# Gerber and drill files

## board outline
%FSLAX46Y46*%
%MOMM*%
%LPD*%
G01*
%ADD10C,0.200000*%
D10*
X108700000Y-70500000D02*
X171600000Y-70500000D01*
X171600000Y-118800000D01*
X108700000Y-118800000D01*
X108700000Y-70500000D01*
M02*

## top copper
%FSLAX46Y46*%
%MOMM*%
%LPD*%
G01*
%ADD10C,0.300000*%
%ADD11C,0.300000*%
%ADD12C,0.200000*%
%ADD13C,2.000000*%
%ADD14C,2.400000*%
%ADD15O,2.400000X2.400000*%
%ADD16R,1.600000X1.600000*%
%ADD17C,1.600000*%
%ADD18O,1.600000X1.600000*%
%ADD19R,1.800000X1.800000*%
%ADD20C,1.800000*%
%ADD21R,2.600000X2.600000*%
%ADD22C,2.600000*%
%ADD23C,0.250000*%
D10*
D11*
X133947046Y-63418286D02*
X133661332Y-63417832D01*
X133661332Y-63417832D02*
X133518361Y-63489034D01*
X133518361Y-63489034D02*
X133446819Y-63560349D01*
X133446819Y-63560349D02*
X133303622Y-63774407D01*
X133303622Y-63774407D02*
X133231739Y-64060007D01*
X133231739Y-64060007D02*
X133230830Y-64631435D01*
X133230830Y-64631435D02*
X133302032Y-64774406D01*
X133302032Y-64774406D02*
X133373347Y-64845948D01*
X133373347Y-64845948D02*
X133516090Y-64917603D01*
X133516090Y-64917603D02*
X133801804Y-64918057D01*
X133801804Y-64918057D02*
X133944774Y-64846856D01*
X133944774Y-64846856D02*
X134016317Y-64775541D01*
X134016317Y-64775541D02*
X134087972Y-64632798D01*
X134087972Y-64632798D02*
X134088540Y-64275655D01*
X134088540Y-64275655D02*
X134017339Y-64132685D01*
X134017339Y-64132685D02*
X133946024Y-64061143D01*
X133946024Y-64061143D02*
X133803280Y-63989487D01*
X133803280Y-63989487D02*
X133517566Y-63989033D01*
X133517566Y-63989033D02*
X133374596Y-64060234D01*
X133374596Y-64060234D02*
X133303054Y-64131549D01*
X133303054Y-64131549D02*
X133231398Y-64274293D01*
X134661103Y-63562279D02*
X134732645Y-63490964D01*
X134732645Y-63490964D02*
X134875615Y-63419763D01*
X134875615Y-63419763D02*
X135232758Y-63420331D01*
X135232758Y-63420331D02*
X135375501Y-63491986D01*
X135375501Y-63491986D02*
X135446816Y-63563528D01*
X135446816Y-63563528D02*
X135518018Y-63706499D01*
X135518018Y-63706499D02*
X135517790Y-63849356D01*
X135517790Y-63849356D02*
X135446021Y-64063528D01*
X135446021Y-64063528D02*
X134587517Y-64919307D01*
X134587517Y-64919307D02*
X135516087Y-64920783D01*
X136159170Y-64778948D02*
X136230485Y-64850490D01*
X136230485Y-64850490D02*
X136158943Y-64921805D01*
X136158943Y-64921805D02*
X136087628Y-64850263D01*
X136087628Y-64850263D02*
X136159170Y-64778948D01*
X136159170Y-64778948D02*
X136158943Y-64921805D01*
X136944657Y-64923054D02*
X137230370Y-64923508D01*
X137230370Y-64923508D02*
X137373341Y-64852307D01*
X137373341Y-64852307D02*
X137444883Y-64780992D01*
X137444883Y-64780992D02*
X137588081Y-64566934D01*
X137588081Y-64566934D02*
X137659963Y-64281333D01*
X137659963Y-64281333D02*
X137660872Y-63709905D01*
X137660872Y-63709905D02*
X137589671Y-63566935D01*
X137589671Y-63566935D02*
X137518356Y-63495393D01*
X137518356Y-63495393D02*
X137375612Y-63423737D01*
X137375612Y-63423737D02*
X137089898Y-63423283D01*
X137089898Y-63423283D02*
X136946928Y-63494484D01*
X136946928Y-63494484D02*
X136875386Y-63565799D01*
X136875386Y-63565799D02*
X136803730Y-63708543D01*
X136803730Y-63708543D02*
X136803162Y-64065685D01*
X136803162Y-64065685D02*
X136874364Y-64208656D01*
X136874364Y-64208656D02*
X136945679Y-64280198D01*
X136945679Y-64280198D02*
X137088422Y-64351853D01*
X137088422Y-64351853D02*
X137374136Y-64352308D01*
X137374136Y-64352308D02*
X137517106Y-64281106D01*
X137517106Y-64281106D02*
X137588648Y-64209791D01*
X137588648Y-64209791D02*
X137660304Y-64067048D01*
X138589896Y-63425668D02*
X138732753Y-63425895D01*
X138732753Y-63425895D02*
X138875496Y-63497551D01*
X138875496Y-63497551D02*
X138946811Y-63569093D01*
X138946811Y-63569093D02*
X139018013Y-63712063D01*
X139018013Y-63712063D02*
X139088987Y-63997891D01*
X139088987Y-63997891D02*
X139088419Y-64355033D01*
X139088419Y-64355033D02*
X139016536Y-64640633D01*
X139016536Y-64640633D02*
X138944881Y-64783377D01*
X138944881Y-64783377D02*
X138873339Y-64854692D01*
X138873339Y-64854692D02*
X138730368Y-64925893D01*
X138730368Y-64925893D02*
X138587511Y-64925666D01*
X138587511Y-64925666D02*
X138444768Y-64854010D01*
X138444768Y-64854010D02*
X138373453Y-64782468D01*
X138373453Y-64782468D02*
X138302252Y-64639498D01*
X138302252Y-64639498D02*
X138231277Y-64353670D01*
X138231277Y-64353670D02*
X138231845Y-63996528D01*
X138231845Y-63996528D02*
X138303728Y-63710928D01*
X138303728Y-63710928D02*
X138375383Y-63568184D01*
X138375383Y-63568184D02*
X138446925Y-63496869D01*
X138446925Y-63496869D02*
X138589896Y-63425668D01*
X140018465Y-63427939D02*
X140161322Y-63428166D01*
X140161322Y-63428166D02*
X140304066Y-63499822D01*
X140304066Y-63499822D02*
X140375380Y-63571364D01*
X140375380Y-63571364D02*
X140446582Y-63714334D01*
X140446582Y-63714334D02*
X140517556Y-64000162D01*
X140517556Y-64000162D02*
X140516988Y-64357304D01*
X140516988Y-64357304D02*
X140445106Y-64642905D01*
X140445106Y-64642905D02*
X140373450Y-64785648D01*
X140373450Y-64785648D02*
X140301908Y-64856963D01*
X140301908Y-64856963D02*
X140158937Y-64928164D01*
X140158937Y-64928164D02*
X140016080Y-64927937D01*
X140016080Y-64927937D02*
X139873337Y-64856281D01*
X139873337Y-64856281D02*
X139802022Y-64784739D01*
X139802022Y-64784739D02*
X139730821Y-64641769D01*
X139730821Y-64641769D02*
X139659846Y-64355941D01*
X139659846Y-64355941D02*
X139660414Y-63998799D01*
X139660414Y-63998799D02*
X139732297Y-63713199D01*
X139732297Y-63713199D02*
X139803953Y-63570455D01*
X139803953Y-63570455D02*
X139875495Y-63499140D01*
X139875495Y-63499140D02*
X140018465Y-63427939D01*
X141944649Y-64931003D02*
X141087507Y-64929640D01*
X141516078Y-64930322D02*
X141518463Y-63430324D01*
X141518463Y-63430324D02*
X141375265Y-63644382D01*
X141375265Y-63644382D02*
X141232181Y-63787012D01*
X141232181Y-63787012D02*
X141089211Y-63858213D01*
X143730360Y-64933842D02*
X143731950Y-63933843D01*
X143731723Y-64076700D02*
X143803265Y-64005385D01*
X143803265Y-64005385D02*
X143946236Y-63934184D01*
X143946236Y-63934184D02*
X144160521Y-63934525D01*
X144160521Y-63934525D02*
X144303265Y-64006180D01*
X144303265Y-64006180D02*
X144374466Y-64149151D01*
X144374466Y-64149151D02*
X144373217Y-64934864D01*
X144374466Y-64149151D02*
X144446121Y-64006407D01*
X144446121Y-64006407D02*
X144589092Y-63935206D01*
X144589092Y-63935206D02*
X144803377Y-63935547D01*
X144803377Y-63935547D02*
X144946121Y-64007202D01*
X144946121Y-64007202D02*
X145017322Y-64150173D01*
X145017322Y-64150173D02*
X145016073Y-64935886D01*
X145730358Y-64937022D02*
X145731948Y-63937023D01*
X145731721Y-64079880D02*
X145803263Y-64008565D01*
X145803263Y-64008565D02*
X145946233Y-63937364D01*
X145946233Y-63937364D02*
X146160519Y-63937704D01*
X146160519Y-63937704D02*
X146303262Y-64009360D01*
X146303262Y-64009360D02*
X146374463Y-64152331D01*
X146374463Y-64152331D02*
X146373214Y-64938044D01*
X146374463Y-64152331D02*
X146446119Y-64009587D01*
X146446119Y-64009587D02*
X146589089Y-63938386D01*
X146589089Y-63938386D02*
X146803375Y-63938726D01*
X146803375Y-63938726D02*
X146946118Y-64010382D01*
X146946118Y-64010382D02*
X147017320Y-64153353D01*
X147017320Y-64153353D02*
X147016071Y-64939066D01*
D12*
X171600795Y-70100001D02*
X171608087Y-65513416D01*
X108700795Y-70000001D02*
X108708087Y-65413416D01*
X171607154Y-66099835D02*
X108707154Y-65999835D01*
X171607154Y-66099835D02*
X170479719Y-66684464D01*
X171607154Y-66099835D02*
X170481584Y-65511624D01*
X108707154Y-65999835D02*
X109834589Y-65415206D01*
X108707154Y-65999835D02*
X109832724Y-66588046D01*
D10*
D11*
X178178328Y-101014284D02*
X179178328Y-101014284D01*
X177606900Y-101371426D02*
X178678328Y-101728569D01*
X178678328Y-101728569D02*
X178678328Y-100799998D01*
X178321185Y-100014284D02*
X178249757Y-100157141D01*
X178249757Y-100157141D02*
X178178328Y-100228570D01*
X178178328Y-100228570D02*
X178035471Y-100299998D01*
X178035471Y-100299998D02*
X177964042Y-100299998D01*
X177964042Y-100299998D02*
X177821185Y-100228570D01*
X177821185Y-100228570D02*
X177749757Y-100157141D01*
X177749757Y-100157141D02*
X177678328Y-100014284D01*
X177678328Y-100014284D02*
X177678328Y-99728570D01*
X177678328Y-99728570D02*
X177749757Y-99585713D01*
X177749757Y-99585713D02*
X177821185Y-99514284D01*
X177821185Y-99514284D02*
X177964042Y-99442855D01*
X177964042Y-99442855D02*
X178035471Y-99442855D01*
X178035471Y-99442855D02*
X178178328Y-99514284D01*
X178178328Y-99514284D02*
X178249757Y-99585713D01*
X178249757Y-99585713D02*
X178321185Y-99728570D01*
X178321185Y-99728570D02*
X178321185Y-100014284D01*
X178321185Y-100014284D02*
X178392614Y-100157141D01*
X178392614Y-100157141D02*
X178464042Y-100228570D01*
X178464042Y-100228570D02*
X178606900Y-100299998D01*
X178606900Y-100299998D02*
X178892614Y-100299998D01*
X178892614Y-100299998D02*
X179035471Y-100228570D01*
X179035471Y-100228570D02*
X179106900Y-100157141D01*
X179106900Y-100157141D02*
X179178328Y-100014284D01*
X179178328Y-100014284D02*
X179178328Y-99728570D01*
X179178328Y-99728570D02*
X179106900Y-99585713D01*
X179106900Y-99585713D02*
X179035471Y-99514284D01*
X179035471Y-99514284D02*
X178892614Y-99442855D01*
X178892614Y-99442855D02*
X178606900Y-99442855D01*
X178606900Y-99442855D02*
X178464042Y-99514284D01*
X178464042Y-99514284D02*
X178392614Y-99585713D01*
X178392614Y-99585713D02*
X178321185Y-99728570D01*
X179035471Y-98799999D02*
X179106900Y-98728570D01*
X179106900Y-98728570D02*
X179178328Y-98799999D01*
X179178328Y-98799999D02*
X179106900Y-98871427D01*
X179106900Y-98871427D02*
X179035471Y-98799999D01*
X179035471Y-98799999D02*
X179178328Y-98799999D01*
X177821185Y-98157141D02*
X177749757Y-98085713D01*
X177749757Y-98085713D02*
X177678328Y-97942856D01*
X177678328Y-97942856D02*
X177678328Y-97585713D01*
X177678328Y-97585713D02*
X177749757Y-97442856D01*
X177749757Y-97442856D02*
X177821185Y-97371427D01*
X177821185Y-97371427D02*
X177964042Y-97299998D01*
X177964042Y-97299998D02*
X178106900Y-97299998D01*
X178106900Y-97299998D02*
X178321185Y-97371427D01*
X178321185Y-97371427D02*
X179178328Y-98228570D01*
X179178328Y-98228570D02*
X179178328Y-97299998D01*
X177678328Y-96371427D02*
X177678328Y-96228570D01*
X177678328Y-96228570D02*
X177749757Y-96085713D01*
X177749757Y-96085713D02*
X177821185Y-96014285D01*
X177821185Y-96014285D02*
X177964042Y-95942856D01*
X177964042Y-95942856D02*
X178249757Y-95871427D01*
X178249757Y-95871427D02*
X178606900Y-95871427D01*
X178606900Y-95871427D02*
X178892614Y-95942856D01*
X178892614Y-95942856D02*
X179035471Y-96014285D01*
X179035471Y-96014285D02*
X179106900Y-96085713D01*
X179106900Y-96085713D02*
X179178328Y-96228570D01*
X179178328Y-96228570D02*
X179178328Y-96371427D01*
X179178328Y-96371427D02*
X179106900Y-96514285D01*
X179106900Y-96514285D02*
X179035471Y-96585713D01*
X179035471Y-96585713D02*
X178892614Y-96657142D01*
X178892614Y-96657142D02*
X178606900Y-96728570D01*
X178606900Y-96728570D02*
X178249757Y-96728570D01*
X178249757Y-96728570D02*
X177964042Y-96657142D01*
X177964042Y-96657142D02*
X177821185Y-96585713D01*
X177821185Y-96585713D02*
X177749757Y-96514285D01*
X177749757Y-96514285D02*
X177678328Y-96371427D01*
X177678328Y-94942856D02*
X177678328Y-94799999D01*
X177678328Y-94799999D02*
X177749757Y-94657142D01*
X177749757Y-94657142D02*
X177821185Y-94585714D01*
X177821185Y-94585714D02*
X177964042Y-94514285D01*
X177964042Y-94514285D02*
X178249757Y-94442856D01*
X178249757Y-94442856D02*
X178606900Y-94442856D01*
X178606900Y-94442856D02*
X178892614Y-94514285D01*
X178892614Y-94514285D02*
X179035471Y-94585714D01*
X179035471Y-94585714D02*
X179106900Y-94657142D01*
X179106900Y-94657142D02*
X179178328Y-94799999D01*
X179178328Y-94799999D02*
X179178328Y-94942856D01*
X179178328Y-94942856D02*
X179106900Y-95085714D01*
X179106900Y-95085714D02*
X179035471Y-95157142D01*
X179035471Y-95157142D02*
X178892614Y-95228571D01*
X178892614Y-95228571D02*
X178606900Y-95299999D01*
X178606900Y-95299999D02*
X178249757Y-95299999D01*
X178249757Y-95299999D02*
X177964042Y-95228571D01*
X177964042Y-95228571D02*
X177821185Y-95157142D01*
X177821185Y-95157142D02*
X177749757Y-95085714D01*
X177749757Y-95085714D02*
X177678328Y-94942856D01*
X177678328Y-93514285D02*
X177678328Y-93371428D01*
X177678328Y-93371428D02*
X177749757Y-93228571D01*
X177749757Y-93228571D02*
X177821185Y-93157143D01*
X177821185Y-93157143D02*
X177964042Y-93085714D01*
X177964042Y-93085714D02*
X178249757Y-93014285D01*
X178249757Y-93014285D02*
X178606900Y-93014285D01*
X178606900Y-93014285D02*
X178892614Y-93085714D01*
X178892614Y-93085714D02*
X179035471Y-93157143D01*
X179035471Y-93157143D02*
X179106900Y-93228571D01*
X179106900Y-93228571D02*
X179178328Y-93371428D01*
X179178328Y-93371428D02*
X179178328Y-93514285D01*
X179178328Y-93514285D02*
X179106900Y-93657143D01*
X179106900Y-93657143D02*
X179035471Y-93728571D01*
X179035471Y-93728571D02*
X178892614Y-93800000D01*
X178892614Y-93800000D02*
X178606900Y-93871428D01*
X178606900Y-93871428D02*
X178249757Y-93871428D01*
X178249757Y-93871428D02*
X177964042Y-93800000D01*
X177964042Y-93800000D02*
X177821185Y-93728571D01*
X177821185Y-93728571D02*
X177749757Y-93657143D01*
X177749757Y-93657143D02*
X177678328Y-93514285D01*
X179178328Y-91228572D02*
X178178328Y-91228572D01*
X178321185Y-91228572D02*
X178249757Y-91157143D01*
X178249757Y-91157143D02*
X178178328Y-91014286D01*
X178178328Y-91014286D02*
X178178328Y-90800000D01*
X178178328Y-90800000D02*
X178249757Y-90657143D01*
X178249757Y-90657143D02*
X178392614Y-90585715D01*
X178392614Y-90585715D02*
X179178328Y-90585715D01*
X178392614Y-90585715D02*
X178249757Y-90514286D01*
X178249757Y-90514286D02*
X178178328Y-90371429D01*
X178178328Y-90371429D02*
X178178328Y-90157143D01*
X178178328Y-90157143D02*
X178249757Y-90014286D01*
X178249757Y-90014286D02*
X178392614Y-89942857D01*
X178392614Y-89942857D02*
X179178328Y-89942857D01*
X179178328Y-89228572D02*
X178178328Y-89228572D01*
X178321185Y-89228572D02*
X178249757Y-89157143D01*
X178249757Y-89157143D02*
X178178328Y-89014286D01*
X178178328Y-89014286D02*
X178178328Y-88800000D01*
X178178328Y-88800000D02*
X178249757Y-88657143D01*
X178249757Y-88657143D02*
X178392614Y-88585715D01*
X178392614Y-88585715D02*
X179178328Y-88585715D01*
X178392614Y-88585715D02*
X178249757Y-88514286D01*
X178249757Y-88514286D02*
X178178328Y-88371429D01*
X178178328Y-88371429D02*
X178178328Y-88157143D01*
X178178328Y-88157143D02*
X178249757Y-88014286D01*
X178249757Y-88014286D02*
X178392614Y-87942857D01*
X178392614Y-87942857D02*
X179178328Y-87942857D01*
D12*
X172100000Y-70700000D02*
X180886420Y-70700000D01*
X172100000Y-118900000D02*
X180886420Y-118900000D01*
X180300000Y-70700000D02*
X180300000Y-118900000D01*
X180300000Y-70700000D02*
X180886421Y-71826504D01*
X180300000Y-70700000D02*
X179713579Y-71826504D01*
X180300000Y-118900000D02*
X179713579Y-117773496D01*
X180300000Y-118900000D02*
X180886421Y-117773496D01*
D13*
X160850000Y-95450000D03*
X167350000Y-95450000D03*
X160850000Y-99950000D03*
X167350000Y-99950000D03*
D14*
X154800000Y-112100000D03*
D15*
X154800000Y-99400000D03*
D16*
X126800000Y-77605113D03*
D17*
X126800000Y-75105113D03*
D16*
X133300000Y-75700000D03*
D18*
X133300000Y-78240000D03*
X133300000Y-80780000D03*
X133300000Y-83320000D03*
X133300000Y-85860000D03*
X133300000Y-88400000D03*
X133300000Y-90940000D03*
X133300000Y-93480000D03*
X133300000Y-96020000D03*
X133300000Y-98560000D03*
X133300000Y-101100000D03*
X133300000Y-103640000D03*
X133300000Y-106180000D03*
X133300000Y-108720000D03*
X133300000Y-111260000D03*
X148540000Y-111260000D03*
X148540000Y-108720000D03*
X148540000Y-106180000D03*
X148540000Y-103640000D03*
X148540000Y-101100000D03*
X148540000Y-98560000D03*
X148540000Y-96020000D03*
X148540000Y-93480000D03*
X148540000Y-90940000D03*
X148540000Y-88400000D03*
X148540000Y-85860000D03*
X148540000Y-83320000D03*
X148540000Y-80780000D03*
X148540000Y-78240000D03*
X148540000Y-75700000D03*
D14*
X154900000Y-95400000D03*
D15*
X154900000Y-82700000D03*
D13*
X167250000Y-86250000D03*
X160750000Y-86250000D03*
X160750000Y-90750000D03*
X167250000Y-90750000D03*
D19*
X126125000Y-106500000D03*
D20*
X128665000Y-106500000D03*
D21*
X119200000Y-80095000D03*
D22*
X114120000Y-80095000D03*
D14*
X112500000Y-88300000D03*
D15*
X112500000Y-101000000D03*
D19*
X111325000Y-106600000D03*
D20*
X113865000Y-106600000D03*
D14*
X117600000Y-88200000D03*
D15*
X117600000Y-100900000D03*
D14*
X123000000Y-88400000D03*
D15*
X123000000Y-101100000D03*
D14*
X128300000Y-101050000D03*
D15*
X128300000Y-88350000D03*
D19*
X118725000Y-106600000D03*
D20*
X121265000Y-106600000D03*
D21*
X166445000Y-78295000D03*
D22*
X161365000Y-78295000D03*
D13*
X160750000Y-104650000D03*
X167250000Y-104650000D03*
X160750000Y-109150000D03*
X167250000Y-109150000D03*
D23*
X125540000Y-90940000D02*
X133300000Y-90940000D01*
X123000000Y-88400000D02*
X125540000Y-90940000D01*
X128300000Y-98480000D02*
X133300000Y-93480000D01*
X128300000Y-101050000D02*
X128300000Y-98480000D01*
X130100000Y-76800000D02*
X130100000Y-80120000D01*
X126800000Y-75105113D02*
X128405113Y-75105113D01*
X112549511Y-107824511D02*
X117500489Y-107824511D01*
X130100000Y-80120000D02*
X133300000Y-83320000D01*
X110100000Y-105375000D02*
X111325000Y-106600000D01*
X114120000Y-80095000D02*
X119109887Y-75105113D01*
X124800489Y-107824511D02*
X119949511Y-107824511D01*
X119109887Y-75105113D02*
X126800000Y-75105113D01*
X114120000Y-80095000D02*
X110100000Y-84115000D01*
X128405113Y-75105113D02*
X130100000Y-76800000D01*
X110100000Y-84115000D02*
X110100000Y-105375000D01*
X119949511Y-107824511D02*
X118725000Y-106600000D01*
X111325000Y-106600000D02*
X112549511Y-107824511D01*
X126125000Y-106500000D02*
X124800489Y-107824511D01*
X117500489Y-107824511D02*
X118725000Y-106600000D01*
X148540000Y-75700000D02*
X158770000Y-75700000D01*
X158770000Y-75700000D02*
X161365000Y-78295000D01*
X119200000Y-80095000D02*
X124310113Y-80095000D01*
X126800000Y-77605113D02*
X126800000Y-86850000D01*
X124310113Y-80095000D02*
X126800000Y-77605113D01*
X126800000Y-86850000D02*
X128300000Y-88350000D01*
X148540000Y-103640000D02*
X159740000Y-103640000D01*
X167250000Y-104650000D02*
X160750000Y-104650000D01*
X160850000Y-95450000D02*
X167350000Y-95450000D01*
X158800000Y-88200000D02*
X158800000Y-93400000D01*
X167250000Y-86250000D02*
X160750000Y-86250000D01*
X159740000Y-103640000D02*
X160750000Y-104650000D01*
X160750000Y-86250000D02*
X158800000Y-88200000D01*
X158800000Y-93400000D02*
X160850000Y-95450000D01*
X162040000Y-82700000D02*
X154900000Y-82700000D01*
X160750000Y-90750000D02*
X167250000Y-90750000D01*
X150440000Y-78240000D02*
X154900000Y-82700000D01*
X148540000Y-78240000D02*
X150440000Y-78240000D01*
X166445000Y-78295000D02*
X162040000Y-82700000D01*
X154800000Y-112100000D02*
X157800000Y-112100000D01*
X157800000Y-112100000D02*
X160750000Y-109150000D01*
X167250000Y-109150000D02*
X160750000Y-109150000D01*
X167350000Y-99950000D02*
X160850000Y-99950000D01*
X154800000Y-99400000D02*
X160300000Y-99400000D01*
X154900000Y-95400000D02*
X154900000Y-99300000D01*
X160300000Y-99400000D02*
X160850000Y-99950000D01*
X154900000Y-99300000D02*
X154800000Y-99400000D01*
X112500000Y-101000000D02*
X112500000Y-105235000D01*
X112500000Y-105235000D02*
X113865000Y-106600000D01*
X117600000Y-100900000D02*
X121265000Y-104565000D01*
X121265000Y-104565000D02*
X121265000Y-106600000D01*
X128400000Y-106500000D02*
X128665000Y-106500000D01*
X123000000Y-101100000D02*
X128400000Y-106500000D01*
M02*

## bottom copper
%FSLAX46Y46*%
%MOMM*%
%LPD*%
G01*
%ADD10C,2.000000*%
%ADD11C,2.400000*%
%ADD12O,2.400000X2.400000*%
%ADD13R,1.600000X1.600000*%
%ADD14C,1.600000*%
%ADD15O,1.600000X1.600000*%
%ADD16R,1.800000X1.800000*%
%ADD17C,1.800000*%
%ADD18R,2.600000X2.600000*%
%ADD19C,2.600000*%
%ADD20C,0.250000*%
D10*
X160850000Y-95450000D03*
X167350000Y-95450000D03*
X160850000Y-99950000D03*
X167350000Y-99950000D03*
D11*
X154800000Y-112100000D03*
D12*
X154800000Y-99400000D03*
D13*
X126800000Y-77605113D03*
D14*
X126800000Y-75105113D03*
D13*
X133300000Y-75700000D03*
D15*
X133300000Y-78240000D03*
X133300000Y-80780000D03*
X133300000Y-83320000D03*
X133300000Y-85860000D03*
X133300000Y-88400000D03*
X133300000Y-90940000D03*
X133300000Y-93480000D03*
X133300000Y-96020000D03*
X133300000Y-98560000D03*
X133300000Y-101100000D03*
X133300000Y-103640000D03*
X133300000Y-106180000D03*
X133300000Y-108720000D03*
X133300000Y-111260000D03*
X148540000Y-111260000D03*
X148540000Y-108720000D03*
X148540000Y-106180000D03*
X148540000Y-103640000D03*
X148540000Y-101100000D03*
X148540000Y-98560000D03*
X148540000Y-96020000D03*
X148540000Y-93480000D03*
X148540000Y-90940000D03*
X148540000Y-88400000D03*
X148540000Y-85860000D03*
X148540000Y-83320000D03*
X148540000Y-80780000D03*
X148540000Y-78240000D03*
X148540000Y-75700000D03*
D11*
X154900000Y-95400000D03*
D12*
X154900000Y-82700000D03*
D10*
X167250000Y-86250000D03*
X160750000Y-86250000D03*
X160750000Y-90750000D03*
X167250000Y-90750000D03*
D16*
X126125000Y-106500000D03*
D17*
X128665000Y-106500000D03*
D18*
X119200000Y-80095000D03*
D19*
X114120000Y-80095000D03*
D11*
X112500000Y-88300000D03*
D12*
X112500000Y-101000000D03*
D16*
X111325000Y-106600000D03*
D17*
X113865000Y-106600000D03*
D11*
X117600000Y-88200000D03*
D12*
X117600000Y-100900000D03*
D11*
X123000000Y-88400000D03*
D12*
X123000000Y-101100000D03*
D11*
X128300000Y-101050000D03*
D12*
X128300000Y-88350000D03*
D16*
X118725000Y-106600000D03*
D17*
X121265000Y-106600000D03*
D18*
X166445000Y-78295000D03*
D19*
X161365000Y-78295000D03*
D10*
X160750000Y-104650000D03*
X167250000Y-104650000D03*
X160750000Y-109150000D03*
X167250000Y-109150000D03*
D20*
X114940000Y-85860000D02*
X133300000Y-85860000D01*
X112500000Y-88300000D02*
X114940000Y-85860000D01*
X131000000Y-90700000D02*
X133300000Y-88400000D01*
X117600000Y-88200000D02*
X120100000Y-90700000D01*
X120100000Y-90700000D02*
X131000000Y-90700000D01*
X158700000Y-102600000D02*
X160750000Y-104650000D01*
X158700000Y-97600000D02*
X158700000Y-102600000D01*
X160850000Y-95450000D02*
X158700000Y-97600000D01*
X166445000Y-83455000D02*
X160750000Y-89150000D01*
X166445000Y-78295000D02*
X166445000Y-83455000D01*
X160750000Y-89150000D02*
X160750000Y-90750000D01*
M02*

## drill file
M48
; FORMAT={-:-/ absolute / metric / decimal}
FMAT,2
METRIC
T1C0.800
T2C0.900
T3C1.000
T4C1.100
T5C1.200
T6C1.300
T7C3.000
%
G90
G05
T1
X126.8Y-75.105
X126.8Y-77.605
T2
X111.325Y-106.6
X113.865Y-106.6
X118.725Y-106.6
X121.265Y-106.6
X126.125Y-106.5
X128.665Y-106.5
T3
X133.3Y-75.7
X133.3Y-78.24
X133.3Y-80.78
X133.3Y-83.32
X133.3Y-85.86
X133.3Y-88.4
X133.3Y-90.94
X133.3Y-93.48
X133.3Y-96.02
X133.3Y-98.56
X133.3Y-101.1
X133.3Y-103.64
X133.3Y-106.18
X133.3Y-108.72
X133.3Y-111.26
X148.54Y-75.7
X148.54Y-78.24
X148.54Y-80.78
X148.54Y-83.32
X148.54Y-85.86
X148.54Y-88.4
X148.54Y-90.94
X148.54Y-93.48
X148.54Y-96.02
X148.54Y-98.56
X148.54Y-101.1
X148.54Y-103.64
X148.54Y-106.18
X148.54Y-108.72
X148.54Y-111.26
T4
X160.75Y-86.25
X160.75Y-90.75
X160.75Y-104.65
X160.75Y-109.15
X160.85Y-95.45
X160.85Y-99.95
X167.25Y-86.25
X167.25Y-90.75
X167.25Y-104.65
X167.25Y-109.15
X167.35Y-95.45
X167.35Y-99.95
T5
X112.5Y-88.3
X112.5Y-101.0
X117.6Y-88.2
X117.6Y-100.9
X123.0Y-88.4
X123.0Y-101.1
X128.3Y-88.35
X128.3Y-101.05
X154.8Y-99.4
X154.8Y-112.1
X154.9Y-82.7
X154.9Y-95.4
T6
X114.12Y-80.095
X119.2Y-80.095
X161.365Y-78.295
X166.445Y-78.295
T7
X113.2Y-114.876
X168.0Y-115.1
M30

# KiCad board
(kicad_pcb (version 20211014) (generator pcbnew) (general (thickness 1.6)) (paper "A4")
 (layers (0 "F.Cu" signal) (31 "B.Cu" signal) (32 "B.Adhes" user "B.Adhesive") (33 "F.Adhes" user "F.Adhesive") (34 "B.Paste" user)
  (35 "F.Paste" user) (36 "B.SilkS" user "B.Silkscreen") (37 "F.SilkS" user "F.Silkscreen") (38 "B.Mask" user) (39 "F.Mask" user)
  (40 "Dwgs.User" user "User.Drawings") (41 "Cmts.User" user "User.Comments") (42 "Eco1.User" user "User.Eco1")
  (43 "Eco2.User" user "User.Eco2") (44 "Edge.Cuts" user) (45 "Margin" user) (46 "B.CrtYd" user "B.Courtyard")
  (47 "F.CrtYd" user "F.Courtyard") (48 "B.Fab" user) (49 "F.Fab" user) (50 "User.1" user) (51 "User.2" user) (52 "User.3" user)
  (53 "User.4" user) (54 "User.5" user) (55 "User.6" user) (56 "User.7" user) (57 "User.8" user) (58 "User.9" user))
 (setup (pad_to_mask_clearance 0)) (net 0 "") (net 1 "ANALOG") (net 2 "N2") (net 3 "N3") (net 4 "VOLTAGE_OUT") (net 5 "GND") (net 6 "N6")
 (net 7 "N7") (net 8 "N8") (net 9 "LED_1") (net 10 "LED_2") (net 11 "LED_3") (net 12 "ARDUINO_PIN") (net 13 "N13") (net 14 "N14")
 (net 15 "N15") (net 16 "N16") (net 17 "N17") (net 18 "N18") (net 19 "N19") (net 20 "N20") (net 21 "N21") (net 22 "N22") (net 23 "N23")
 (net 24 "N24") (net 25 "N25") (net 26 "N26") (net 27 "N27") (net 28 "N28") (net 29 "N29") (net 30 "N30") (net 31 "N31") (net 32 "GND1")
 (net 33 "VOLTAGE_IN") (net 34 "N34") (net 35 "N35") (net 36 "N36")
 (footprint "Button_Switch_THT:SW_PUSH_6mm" (layer "F.Cu") (at 160.85 95.45)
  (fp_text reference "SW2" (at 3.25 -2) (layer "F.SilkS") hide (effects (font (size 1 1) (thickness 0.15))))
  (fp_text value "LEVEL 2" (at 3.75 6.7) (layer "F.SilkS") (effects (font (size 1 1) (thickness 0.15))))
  (pad "1" thru_hole circle (at 0 0 90) (size 2 2) (drill 1.1) (layers *.Cu *.Mask) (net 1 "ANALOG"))
  (pad "1" thru_hole circle (at 6.5 0 90) (size 2 2) (drill 1.1) (layers *.Cu *.Mask) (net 1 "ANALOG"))
  (pad "2" thru_hole circle (at 0 4.5 90) (size 2 2) (drill 1.1) (layers *.Cu *.Mask) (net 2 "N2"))
  (pad "2" thru_hole circle (at 6.5 4.5 90) (size 2 2) (drill 1.1) (layers *.Cu *.Mask) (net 2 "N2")))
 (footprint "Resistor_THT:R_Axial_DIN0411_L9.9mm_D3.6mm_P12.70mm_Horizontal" (layer "F.Cu") (at 154.8 112.1 90)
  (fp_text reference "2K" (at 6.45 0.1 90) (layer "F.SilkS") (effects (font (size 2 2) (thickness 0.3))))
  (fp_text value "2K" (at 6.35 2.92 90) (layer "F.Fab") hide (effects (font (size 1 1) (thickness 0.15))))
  (pad "1" thru_hole circle (at 0 0 90) (size 2.4 2.4) (drill 1.2) (layers *.Cu *.Mask) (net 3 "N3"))
  (pad "2" thru_hole oval (at 12.7 0 90) (size 2.4 2.4) (drill 1.2) (layers *.Cu *.Mask) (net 2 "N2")))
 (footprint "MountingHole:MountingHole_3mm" (layer "F.Cu") (at 168 115.1)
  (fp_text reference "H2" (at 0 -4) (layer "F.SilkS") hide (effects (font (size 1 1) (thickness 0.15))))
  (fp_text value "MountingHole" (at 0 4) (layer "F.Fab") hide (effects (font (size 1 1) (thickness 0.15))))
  (pad "" np_thru_hole circle (at 0 0) (size 3 3) (drill 3) (layers *.Cu *.Mask)))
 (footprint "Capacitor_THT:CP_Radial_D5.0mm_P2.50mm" (layer "F.Cu") (at 126.8 77.605113 90)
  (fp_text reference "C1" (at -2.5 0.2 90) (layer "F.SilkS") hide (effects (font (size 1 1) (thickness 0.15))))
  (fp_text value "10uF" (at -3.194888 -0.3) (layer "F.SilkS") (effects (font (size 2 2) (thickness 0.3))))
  (pad "1" thru_hole rect (at 0 0 90) (size 1.6 1.6) (drill 0.8) (layers *.Cu *.Mask) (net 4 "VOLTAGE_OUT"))
  (pad "2" thru_hole circle (at 2.5 0 90) (size 1.6 1.6) (drill 0.8) (layers *.Cu *.Mask) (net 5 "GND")))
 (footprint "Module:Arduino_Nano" (layer "F.Cu") (at 133.3 75.7)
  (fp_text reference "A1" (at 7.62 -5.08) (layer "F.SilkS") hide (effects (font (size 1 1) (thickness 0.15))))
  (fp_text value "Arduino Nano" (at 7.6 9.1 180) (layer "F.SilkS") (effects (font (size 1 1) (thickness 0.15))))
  (pad "1" thru_hole rect (at 0 0) (size 1.6 1.6) (drill 1) (layers *.Cu *.Mask) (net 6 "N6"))
  (pad "2" thru_hole oval (at 0 2.54) (size 1.6 1.6) (drill 1) (layers *.Cu *.Mask) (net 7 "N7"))
  (pad "3" thru_hole oval (at 0 5.08) (size 1.6 1.6) (drill 1) (layers *.Cu *.Mask) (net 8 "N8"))
  (pad "4" thru_hole oval (at 0 7.62) (size 1.6 1.6) (drill 1) (layers *.Cu *.Mask) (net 5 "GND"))
  (pad "5" thru_hole oval (at 0 10.16) (size 1.6 1.6) (drill 1) (layers *.Cu *.Mask) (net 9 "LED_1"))
  (pad "6" thru_hole oval (at 0 12.7) (size 1.6 1.6) (drill 1) (layers *.Cu *.Mask) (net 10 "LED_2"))
  (pad "7" thru_hole oval (at 0 15.24) (size 1.6 1.6) (drill 1) (layers *.Cu *.Mask) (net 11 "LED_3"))
  (pad "8" thru_hole oval (at 0 17.78) (size 1.6 1.6) (drill 1) (layers *.Cu *.Mask) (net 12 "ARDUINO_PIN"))
  (pad "9" thru_hole oval (at 0 20.32) (size 1.6 1.6) (drill 1) (layers *.Cu *.Mask) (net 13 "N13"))
  (pad "10" thru_hole oval (at 0 22.86) (size 1.6 1.6) (drill 1) (layers *.Cu *.Mask) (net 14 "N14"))
  (pad "11" thru_hole oval (at 0 25.4) (size 1.6 1.6) (drill 1) (layers *.Cu *.Mask) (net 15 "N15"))
  (pad "12" thru_hole oval (at 0 27.94) (size 1.6 1.6) (drill 1) (layers *.Cu *.Mask) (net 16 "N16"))
  (pad "13" thru_hole oval (at 0 30.48) (size 1.6 1.6) (drill 1) (layers *.Cu *.Mask) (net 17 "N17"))
  (pad "14" thru_hole oval (at 0 33.02) (size 1.6 1.6) (drill 1) (layers *.Cu *.Mask) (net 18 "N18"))
  (pad "15" thru_hole oval (at 0 35.56) (size 1.6 1.6) (drill 1) (layers *.Cu *.Mask) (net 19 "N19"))
  (pad "16" thru_hole oval (at 15.24 35.56) (size 1.6 1.6) (drill 1) (layers *.Cu *.Mask) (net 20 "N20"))
  (pad "17" thru_hole oval (at 15.24 33.02) (size 1.6 1.6) (drill 1) (layers *.Cu *.Mask) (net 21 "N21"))
  (pad "18" thru_hole oval (at 15.24 30.48) (size 1.6 1.6) (drill 1) (layers *.Cu *.Mask) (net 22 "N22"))
  (pad "19" thru_hole oval (at 15.24 27.94) (size 1.6 1.6) (drill 1) (layers *.Cu *.Mask) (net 1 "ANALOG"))
  (pad "20" thru_hole oval (at 15.24 25.4) (size 1.6 1.6) (drill 1) (layers *.Cu *.Mask) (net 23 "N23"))
  (pad "21" thru_hole oval (at 15.24 22.86) (size 1.6 1.6) (drill 1) (layers *.Cu *.Mask) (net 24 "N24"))
  (pad "22" thru_hole oval (at 15.24 20.32) (size 1.6 1.6) (drill 1) (layers *.Cu *.Mask) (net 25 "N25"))
  (pad "23" thru_hole oval (at 15.24 17.78) (size 1.6 1.6) (drill 1) (layers *.Cu *.Mask) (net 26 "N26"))
  (pad "24" thru_hole oval (at 15.24 15.24) (size 1.6 1.6) (drill 1) (layers *.Cu *.Mask) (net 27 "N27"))
  (pad "25" thru_hole oval (at 15.24 12.7) (size 1.6 1.6) (drill 1) (layers *.Cu *.Mask) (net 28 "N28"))
  (pad "26" thru_hole oval (at 15.24 10.16) (size 1.6 1.6) (drill 1) (layers *.Cu *.Mask) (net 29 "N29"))
  (pad "27" thru_hole oval (at 15.24 7.62) (size 1.6 1.6) (drill 1) (layers *.Cu *.Mask) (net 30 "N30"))
  (pad "28" thru_hole oval (at 15.24 5.08) (size 1.6 1.6) (drill 1) (layers *.Cu *.Mask) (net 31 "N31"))
  (pad "29" thru_hole oval (at 15.24 2.54) (size 1.6 1.6) (drill 1) (layers *.Cu *.Mask) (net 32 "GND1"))
  (pad "30" thru_hole oval (at 15.24 0) (size 1.6 1.6) (drill 1) (layers *.Cu *.Mask) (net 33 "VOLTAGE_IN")))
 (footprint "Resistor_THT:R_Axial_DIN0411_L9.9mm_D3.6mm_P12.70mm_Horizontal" (layer "F.Cu") (at 154.9 95.4 90)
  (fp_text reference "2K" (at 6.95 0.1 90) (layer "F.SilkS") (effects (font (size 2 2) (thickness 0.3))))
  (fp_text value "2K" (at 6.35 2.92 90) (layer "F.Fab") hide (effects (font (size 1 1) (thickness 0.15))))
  (pad "1" thru_hole circle (at 0 0 90) (size 2.4 2.4) (drill 1.2) (layers *.Cu *.Mask) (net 2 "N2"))
  (pad "2" thru_hole oval (at 12.7 0 90) (size 2.4 2.4) (drill 1.2) (layers *.Cu *.Mask) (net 32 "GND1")))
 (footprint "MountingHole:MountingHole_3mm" (layer "F.Cu") (at 113.2 114.876494)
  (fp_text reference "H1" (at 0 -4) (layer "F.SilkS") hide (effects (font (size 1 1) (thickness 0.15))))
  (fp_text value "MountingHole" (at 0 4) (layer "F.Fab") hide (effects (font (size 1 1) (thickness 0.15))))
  (pad "" np_thru_hole circle (at 0 0) (size 3 3) (drill 3) (layers *.Cu *.Mask)))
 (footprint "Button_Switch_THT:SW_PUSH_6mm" (layer "F.Cu") (at 160.75 86.25)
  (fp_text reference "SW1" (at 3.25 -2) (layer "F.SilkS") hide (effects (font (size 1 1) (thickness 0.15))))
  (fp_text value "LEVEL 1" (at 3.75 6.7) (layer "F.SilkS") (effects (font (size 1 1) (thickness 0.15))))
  (pad "1" thru_hole circle (at 6.5 0 90) (size 2 2) (drill 1.1) (layers *.Cu *.Mask) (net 1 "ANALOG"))
  (pad "1" thru_hole circle (at 0 0 90) (size 2 2) (drill 1.1) (layers *.Cu *.Mask) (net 1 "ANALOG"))
  (pad "2" thru_hole circle (at 0 4.5 90) (size 2 2) (drill 1.1) (layers *.Cu *.Mask) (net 32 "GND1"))
  (pad "2" thru_hole circle (at 6.5 4.5 90) (size 2 2) (drill 1.1) (layers *.Cu *.Mask) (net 32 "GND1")))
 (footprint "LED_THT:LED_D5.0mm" (layer "F.Cu") (at 126.125 106.5)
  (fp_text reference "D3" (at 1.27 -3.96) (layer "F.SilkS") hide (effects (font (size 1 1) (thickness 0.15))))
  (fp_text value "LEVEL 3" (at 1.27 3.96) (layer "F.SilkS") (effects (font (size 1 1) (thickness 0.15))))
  (pad "1" thru_hole rect (at 0 0) (size 1.8 1.8) (drill 0.9) (layers *.Cu *.Mask) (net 5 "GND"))
  (pad "2" thru_hole circle (at 2.54 0) (size 1.8 1.8) (drill 0.9) (layers *.Cu *.Mask) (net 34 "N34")))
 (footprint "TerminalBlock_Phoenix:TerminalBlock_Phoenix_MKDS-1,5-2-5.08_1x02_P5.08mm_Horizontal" (layer "F.Cu") (at 119.2 80.095 180)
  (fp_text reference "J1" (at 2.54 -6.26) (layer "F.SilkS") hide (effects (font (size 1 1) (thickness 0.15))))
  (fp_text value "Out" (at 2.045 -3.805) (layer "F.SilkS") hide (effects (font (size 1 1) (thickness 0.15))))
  (pad "1" thru_hole rect (at 0 0 180) (size 2.6 2.6) (drill 1.3) (layers *.Cu *.Mask) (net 4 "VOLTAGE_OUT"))
  (pad "2" thru_hole circle (at 5.08 0 180) (size 2.6 2.6) (drill 1.3) (layers *.Cu *.Mask) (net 5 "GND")))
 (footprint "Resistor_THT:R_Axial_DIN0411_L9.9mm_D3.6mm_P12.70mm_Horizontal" (layer "F.Cu") (at 112.5 88.3 -90)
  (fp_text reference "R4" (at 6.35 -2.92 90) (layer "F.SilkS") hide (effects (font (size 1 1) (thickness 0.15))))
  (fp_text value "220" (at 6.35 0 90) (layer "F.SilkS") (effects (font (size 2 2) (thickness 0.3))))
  (pad "1" thru_hole circle (at 0 0 270) (size 2.4 2.4) (drill 1.2) (layers *.Cu *.Mask) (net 9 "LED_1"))
  (pad "2" thru_hole oval (at 12.7 0 270) (size 2.4 2.4) (drill 1.2) (layers *.Cu *.Mask) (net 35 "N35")))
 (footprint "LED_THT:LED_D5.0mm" (layer "F.Cu") (at 111.325 106.6)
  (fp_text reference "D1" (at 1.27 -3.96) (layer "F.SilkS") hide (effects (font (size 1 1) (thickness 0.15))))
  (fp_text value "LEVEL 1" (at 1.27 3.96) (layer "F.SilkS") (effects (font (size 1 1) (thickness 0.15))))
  (pad "1" thru_hole rect (at 0 0) (size 1.8 1.8) (drill 0.9) (layers *.Cu *.Mask) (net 5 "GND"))
  (pad "2" thru_hole circle (at 2.54 0) (size 1.8 1.8) (drill 0.9) (layers *.Cu *.Mask) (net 35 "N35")))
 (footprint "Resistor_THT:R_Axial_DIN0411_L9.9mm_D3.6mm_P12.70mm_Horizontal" (layer "F.Cu") (at 117.6 88.2 -90)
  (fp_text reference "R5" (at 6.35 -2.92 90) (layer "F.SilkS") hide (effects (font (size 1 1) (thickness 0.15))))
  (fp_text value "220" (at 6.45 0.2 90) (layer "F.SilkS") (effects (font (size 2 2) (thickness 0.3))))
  (pad "1" thru_hole circle (at 0 0 270) (size 2.4 2.4) (drill 1.2) (layers *.Cu *.Mask) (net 10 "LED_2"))
  (pad "2" thru_hole oval (at 12.7 0 270) (size 2.4 2.4) (drill 1.2) (layers *.Cu *.Mask) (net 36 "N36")))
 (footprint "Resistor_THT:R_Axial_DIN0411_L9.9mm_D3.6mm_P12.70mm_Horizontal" (layer "F.Cu") (at 123 88.4 -90)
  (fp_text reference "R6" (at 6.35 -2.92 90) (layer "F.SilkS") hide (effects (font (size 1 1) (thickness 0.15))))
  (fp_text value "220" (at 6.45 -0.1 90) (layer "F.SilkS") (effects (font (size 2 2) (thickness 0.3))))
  (pad "1" thru_hole circle (at 0 0 270) (size 2.4 2.4) (drill 1.2) (layers *.Cu *.Mask) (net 11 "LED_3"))
  (pad "2" thru_hole oval (at 12.7 0 270) (size 2.4 2.4) (drill 1.2) (layers *.Cu *.Mask) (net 34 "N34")))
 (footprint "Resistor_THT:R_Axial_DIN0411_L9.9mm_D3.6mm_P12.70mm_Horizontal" (layer "F.Cu") (at 128.3 101.05 90)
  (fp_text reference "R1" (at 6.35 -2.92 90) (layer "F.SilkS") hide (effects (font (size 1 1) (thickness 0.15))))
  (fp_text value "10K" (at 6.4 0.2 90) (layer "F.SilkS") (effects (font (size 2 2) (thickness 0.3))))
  (pad "1" thru_hole circle (at 0 0 90) (size 2.4 2.4) (drill 1.2) (layers *.Cu *.Mask) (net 12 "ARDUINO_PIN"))
  (pad "2" thru_hole oval (at 12.7 0 90) (size 2.4 2.4) (drill 1.2) (layers *.Cu *.Mask) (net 4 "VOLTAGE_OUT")))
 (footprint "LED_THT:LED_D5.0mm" (layer "F.Cu") (at 118.725 106.6)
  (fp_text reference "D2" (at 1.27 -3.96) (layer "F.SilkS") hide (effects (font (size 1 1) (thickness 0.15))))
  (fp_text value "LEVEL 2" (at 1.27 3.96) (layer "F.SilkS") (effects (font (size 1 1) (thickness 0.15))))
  (pad "1" thru_hole rect (at 0 0) (size 1.8 1.8) (drill 0.9) (layers *.Cu *.Mask) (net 5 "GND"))
  (pad "2" thru_hole circle (at 2.54 0) (size 1.8 1.8) (drill 0.9) (layers *.Cu *.Mask) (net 36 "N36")))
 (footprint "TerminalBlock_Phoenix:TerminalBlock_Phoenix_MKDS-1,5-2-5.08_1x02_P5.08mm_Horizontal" (layer "F.Cu") (at 166.445 78.295 180)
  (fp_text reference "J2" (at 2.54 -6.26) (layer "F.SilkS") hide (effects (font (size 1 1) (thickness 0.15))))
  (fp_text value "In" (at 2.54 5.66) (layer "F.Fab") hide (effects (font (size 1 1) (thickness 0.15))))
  (pad "1" thru_hole rect (at 0 0 180) (size 2.6 2.6) (drill 1.3) (layers *.Cu *.Mask) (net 32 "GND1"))
  (pad "2" thru_hole circle (at 5.08 0 180) (size 2.6 2.6) (drill 1.3) (layers *.Cu *.Mask) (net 33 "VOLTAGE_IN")))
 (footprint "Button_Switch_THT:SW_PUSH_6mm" (layer "F.Cu") (at 160.75 104.65)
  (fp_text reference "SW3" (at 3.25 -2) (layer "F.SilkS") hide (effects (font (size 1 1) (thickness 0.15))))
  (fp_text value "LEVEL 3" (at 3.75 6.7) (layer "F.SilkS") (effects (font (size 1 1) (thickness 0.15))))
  (pad "1" thru_hole circle (at 0 0 90) (size 2 2) (drill 1.1) (layers *.Cu *.Mask) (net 1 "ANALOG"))
  (pad "1" thru_hole circle (at 6.5 0 90) (size 2 2) (drill 1.1) (layers *.Cu *.Mask) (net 1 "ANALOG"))
  (pad "2" thru_hole circle (at 0 4.5 90) (size 2 2) (drill 1.1) (layers *.Cu *.Mask) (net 3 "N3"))
  (pad "2" thru_hole circle (at 6.5 4.5 90) (size 2 2) (drill 1.1) (layers *.Cu *.Mask) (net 3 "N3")))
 (gr_rect (start 108.7 70.5) (end 171.6 118.8) (layer "Edge.Cuts") (width 0.2) (fill none))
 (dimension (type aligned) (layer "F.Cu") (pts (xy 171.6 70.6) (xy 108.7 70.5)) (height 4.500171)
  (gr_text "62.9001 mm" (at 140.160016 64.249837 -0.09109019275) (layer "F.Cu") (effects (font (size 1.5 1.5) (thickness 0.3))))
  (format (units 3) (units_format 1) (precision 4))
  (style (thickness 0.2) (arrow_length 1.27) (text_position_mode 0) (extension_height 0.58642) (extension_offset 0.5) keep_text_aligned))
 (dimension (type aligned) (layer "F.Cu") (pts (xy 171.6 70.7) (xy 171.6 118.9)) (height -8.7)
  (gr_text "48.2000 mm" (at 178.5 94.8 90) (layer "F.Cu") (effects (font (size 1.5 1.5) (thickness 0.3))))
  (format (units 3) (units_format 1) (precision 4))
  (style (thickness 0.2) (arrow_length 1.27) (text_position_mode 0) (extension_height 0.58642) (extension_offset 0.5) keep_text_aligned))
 (segment (start 114.94 85.86) (end 133.3 85.86) (width 0.25) (layer "B.Cu") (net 9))
 (segment (start 112.5 88.3) (end 114.94 85.86) (width 0.25) (layer "B.Cu") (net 9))
 (segment (start 131 90.7) (end 133.3 88.4) (width 0.25) (layer "B.Cu") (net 10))
 (segment (start 117.6 88.2) (end 120.1 90.7) (width 0.25) (layer "B.Cu") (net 10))
 (segment (start 120.1 90.7) (end 131 90.7) (width 0.25) (layer "B.Cu") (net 10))
 (segment (start 125.54 90.94) (end 133.3 90.94) (width 0.25) (layer "F.Cu") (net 11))
 (segment (start 123 88.4) (end 125.54 90.94) (width 0.25) (layer "F.Cu") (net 11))
 (segment (start 128.3 98.48) (end 133.3 93.48) (width 0.25) (layer "F.Cu") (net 12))
 (segment (start 128.3 101.05) (end 128.3 98.48) (width 0.25) (layer "F.Cu") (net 12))
 (segment (start 130.1 76.8) (end 130.1 80.12) (width 0.25) (layer "F.Cu") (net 5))
 (segment (start 126.8 75.105113) (end 128.405113 75.105113) (width 0.25) (layer "F.Cu") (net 5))
 (segment (start 112.549511 107.824511) (end 117.500489 107.824511) (width 0.25) (layer "F.Cu") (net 5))
 (segment (start 130.1 80.12) (end 133.3 83.32) (width 0.25) (layer "F.Cu") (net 5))
 (segment (start 110.1 105.375) (end 111.325 106.6) (width 0.25) (layer "F.Cu") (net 5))
 (segment (start 114.12 80.095) (end 119.109887 75.105113) (width 0.25) (layer "F.Cu") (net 5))
 (segment (start 124.800489 107.824511) (end 119.949511 107.824511) (width 0.25) (layer "F.Cu") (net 5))
 (segment (start 119.109887 75.105113) (end 126.8 75.105113) (width 0.25) (layer "F.Cu") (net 5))
 (segment (start 114.12 80.095) (end 110.1 84.115) (width 0.25) (layer "F.Cu") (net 5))
 (segment (start 128.405113 75.105113) (end 130.1 76.8) (width 0.25) (layer "F.Cu") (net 5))
 (segment (start 110.1 84.115) (end 110.1 105.375) (width 0.25) (layer "F.Cu") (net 5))
 (segment (start 119.949511 107.824511) (end 118.725 106.6) (width 0.25) (layer "F.Cu") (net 5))
 (segment (start 111.325 106.6) (end 112.549511 107.824511) (width 0.25) (layer "F.Cu") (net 5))
 (segment (start 126.125 106.5) (end 124.800489 107.824511) (width 0.25) (layer "F.Cu") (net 5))
 (segment (start 117.500489 107.824511) (end 118.725 106.6) (width 0.25) (layer "F.Cu") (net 5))
 (segment (start 148.54 75.7) (end 158.77 75.7) (width 0.25) (layer "F.Cu") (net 33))
 (segment (start 158.77 75.7) (end 161.365 78.295) (width 0.25) (layer "F.Cu") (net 33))
 (segment (start 119.2 80.095) (end 124.310113 80.095) (width 0.25) (layer "F.Cu") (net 4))
 (segment (start 126.8 77.605113) (end 126.8 86.85) (width 0.25) (layer "F.Cu") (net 4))
 (segment (start 124.310113 80.095) (end 126.8 77.605113) (width 0.25) (layer "F.Cu") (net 4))
 (segment (start 126.8 86.85) (end 128.3 88.35) (width 0.25) (layer "F.Cu") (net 4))
 (segment (start 148.54 103.64) (end 159.74 103.64) (width 0.25) (layer "F.Cu") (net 1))
 (segment (start 167.25 104.65) (end 160.75 104.65) (width 0.25) (layer "F.Cu") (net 1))
 (segment (start 160.85 95.45) (end 167.35 95.45) (width 0.25) (layer "F.Cu") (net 1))
 (segment (start 158.8 88.2) (end 158.8 93.4) (width 0.25) (layer "F.Cu") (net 1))
 (segment (start 167.25 86.25) (end 160.75 86.25) (width 0.25) (layer "F.Cu") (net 1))
 (segment (start 159.74 103.64) (end 160.75 104.65) (width 0.25) (layer "F.Cu") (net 1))
 (segment (start 160.75 86.25) (end 158.8 88.2) (width 0.25) (layer "F.Cu") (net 1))
 (segment (start 158.8 93.4) (end 160.85 95.45) (width 0.25) (layer "F.Cu") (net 1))
 (segment (start 158.7 102.6) (end 160.75 104.65) (width 0.25) (layer "B.Cu") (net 1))
 (segment (start 158.7 97.6) (end 158.7 102.6) (width 0.25) (layer "B.Cu") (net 1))
 (segment (start 160.85 95.45) (end 158.7 97.6) (width 0.25) (layer "B.Cu") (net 1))
 (segment (start 162.04 82.7) (end 154.9 82.7) (width 0.25) (layer "F.Cu") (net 32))
 (segment (start 160.75 90.75) (end 167.25 90.75) (width 0.25) (layer "F.Cu") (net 32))
 (segment (start 150.44 78.24) (end 154.9 82.7) (width 0.25) (layer "F.Cu") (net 32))
 (segment (start 148.54 78.24) (end 150.44 78.24) (width 0.25) (layer "F.Cu") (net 32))
 (segment (start 166.445 78.295) (end 162.04 82.7) (width 0.25) (layer "F.Cu") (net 32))
 (segment (start 166.445 83.455) (end 160.75 89.15) (width 0.25) (layer "B.Cu") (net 32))
 (segment (start 166.445 78.295) (end 166.445 83.455) (width 0.25) (layer "B.Cu") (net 32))
 (segment (start 160.75 89.15) (end 160.75 90.75) (width 0.25) (layer "B.Cu") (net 32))
 (segment (start 154.8 112.1) (end 157.8 112.1) (width 0.25) (layer "F.Cu") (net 3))
 (segment (start 157.8 112.1) (end 160.75 109.15) (width 0.25) (layer "F.Cu") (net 3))
 (segment (start 167.25 109.15) (end 160.75 109.15) (width 0.25) (layer "F.Cu") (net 3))
 (segment (start 167.35 99.95) (end 160.85 99.95) (width 0.25) (layer "F.Cu") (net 2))
 (segment (start 154.8 99.4) (end 160.3 99.4) (width 0.25) (layer "F.Cu") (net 2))
 (segment (start 154.9 95.4) (end 154.9 99.3) (width 0.25) (layer "F.Cu") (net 2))
 (segment (start 160.3 99.4) (end 160.85 99.95) (width 0.25) (layer "F.Cu") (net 2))
 (segment (start 154.9 99.3) (end 154.8 99.4) (width 0.25) (layer "F.Cu") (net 2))
 (segment (start 112.5 101) (end 112.5 105.235) (width 0.25) (layer "F.Cu") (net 35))
 (segment (start 112.5 105.235) (end 113.865 106.6) (width 0.25) (layer "F.Cu") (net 35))
 (segment (start 117.6 100.9) (end 121.265 104.565) (width 0.25) (layer "F.Cu") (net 36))
 (segment (start 121.265 104.565) (end 121.265 106.6) (width 0.25) (layer "F.Cu") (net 36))
 (segment (start 128.4 106.5) (end 128.665 106.5) (width 0.25) (layer "F.Cu") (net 34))
 (segment (start 123 101.1) (end 128.4 106.5) (width 0.25) (layer "F.Cu") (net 34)))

